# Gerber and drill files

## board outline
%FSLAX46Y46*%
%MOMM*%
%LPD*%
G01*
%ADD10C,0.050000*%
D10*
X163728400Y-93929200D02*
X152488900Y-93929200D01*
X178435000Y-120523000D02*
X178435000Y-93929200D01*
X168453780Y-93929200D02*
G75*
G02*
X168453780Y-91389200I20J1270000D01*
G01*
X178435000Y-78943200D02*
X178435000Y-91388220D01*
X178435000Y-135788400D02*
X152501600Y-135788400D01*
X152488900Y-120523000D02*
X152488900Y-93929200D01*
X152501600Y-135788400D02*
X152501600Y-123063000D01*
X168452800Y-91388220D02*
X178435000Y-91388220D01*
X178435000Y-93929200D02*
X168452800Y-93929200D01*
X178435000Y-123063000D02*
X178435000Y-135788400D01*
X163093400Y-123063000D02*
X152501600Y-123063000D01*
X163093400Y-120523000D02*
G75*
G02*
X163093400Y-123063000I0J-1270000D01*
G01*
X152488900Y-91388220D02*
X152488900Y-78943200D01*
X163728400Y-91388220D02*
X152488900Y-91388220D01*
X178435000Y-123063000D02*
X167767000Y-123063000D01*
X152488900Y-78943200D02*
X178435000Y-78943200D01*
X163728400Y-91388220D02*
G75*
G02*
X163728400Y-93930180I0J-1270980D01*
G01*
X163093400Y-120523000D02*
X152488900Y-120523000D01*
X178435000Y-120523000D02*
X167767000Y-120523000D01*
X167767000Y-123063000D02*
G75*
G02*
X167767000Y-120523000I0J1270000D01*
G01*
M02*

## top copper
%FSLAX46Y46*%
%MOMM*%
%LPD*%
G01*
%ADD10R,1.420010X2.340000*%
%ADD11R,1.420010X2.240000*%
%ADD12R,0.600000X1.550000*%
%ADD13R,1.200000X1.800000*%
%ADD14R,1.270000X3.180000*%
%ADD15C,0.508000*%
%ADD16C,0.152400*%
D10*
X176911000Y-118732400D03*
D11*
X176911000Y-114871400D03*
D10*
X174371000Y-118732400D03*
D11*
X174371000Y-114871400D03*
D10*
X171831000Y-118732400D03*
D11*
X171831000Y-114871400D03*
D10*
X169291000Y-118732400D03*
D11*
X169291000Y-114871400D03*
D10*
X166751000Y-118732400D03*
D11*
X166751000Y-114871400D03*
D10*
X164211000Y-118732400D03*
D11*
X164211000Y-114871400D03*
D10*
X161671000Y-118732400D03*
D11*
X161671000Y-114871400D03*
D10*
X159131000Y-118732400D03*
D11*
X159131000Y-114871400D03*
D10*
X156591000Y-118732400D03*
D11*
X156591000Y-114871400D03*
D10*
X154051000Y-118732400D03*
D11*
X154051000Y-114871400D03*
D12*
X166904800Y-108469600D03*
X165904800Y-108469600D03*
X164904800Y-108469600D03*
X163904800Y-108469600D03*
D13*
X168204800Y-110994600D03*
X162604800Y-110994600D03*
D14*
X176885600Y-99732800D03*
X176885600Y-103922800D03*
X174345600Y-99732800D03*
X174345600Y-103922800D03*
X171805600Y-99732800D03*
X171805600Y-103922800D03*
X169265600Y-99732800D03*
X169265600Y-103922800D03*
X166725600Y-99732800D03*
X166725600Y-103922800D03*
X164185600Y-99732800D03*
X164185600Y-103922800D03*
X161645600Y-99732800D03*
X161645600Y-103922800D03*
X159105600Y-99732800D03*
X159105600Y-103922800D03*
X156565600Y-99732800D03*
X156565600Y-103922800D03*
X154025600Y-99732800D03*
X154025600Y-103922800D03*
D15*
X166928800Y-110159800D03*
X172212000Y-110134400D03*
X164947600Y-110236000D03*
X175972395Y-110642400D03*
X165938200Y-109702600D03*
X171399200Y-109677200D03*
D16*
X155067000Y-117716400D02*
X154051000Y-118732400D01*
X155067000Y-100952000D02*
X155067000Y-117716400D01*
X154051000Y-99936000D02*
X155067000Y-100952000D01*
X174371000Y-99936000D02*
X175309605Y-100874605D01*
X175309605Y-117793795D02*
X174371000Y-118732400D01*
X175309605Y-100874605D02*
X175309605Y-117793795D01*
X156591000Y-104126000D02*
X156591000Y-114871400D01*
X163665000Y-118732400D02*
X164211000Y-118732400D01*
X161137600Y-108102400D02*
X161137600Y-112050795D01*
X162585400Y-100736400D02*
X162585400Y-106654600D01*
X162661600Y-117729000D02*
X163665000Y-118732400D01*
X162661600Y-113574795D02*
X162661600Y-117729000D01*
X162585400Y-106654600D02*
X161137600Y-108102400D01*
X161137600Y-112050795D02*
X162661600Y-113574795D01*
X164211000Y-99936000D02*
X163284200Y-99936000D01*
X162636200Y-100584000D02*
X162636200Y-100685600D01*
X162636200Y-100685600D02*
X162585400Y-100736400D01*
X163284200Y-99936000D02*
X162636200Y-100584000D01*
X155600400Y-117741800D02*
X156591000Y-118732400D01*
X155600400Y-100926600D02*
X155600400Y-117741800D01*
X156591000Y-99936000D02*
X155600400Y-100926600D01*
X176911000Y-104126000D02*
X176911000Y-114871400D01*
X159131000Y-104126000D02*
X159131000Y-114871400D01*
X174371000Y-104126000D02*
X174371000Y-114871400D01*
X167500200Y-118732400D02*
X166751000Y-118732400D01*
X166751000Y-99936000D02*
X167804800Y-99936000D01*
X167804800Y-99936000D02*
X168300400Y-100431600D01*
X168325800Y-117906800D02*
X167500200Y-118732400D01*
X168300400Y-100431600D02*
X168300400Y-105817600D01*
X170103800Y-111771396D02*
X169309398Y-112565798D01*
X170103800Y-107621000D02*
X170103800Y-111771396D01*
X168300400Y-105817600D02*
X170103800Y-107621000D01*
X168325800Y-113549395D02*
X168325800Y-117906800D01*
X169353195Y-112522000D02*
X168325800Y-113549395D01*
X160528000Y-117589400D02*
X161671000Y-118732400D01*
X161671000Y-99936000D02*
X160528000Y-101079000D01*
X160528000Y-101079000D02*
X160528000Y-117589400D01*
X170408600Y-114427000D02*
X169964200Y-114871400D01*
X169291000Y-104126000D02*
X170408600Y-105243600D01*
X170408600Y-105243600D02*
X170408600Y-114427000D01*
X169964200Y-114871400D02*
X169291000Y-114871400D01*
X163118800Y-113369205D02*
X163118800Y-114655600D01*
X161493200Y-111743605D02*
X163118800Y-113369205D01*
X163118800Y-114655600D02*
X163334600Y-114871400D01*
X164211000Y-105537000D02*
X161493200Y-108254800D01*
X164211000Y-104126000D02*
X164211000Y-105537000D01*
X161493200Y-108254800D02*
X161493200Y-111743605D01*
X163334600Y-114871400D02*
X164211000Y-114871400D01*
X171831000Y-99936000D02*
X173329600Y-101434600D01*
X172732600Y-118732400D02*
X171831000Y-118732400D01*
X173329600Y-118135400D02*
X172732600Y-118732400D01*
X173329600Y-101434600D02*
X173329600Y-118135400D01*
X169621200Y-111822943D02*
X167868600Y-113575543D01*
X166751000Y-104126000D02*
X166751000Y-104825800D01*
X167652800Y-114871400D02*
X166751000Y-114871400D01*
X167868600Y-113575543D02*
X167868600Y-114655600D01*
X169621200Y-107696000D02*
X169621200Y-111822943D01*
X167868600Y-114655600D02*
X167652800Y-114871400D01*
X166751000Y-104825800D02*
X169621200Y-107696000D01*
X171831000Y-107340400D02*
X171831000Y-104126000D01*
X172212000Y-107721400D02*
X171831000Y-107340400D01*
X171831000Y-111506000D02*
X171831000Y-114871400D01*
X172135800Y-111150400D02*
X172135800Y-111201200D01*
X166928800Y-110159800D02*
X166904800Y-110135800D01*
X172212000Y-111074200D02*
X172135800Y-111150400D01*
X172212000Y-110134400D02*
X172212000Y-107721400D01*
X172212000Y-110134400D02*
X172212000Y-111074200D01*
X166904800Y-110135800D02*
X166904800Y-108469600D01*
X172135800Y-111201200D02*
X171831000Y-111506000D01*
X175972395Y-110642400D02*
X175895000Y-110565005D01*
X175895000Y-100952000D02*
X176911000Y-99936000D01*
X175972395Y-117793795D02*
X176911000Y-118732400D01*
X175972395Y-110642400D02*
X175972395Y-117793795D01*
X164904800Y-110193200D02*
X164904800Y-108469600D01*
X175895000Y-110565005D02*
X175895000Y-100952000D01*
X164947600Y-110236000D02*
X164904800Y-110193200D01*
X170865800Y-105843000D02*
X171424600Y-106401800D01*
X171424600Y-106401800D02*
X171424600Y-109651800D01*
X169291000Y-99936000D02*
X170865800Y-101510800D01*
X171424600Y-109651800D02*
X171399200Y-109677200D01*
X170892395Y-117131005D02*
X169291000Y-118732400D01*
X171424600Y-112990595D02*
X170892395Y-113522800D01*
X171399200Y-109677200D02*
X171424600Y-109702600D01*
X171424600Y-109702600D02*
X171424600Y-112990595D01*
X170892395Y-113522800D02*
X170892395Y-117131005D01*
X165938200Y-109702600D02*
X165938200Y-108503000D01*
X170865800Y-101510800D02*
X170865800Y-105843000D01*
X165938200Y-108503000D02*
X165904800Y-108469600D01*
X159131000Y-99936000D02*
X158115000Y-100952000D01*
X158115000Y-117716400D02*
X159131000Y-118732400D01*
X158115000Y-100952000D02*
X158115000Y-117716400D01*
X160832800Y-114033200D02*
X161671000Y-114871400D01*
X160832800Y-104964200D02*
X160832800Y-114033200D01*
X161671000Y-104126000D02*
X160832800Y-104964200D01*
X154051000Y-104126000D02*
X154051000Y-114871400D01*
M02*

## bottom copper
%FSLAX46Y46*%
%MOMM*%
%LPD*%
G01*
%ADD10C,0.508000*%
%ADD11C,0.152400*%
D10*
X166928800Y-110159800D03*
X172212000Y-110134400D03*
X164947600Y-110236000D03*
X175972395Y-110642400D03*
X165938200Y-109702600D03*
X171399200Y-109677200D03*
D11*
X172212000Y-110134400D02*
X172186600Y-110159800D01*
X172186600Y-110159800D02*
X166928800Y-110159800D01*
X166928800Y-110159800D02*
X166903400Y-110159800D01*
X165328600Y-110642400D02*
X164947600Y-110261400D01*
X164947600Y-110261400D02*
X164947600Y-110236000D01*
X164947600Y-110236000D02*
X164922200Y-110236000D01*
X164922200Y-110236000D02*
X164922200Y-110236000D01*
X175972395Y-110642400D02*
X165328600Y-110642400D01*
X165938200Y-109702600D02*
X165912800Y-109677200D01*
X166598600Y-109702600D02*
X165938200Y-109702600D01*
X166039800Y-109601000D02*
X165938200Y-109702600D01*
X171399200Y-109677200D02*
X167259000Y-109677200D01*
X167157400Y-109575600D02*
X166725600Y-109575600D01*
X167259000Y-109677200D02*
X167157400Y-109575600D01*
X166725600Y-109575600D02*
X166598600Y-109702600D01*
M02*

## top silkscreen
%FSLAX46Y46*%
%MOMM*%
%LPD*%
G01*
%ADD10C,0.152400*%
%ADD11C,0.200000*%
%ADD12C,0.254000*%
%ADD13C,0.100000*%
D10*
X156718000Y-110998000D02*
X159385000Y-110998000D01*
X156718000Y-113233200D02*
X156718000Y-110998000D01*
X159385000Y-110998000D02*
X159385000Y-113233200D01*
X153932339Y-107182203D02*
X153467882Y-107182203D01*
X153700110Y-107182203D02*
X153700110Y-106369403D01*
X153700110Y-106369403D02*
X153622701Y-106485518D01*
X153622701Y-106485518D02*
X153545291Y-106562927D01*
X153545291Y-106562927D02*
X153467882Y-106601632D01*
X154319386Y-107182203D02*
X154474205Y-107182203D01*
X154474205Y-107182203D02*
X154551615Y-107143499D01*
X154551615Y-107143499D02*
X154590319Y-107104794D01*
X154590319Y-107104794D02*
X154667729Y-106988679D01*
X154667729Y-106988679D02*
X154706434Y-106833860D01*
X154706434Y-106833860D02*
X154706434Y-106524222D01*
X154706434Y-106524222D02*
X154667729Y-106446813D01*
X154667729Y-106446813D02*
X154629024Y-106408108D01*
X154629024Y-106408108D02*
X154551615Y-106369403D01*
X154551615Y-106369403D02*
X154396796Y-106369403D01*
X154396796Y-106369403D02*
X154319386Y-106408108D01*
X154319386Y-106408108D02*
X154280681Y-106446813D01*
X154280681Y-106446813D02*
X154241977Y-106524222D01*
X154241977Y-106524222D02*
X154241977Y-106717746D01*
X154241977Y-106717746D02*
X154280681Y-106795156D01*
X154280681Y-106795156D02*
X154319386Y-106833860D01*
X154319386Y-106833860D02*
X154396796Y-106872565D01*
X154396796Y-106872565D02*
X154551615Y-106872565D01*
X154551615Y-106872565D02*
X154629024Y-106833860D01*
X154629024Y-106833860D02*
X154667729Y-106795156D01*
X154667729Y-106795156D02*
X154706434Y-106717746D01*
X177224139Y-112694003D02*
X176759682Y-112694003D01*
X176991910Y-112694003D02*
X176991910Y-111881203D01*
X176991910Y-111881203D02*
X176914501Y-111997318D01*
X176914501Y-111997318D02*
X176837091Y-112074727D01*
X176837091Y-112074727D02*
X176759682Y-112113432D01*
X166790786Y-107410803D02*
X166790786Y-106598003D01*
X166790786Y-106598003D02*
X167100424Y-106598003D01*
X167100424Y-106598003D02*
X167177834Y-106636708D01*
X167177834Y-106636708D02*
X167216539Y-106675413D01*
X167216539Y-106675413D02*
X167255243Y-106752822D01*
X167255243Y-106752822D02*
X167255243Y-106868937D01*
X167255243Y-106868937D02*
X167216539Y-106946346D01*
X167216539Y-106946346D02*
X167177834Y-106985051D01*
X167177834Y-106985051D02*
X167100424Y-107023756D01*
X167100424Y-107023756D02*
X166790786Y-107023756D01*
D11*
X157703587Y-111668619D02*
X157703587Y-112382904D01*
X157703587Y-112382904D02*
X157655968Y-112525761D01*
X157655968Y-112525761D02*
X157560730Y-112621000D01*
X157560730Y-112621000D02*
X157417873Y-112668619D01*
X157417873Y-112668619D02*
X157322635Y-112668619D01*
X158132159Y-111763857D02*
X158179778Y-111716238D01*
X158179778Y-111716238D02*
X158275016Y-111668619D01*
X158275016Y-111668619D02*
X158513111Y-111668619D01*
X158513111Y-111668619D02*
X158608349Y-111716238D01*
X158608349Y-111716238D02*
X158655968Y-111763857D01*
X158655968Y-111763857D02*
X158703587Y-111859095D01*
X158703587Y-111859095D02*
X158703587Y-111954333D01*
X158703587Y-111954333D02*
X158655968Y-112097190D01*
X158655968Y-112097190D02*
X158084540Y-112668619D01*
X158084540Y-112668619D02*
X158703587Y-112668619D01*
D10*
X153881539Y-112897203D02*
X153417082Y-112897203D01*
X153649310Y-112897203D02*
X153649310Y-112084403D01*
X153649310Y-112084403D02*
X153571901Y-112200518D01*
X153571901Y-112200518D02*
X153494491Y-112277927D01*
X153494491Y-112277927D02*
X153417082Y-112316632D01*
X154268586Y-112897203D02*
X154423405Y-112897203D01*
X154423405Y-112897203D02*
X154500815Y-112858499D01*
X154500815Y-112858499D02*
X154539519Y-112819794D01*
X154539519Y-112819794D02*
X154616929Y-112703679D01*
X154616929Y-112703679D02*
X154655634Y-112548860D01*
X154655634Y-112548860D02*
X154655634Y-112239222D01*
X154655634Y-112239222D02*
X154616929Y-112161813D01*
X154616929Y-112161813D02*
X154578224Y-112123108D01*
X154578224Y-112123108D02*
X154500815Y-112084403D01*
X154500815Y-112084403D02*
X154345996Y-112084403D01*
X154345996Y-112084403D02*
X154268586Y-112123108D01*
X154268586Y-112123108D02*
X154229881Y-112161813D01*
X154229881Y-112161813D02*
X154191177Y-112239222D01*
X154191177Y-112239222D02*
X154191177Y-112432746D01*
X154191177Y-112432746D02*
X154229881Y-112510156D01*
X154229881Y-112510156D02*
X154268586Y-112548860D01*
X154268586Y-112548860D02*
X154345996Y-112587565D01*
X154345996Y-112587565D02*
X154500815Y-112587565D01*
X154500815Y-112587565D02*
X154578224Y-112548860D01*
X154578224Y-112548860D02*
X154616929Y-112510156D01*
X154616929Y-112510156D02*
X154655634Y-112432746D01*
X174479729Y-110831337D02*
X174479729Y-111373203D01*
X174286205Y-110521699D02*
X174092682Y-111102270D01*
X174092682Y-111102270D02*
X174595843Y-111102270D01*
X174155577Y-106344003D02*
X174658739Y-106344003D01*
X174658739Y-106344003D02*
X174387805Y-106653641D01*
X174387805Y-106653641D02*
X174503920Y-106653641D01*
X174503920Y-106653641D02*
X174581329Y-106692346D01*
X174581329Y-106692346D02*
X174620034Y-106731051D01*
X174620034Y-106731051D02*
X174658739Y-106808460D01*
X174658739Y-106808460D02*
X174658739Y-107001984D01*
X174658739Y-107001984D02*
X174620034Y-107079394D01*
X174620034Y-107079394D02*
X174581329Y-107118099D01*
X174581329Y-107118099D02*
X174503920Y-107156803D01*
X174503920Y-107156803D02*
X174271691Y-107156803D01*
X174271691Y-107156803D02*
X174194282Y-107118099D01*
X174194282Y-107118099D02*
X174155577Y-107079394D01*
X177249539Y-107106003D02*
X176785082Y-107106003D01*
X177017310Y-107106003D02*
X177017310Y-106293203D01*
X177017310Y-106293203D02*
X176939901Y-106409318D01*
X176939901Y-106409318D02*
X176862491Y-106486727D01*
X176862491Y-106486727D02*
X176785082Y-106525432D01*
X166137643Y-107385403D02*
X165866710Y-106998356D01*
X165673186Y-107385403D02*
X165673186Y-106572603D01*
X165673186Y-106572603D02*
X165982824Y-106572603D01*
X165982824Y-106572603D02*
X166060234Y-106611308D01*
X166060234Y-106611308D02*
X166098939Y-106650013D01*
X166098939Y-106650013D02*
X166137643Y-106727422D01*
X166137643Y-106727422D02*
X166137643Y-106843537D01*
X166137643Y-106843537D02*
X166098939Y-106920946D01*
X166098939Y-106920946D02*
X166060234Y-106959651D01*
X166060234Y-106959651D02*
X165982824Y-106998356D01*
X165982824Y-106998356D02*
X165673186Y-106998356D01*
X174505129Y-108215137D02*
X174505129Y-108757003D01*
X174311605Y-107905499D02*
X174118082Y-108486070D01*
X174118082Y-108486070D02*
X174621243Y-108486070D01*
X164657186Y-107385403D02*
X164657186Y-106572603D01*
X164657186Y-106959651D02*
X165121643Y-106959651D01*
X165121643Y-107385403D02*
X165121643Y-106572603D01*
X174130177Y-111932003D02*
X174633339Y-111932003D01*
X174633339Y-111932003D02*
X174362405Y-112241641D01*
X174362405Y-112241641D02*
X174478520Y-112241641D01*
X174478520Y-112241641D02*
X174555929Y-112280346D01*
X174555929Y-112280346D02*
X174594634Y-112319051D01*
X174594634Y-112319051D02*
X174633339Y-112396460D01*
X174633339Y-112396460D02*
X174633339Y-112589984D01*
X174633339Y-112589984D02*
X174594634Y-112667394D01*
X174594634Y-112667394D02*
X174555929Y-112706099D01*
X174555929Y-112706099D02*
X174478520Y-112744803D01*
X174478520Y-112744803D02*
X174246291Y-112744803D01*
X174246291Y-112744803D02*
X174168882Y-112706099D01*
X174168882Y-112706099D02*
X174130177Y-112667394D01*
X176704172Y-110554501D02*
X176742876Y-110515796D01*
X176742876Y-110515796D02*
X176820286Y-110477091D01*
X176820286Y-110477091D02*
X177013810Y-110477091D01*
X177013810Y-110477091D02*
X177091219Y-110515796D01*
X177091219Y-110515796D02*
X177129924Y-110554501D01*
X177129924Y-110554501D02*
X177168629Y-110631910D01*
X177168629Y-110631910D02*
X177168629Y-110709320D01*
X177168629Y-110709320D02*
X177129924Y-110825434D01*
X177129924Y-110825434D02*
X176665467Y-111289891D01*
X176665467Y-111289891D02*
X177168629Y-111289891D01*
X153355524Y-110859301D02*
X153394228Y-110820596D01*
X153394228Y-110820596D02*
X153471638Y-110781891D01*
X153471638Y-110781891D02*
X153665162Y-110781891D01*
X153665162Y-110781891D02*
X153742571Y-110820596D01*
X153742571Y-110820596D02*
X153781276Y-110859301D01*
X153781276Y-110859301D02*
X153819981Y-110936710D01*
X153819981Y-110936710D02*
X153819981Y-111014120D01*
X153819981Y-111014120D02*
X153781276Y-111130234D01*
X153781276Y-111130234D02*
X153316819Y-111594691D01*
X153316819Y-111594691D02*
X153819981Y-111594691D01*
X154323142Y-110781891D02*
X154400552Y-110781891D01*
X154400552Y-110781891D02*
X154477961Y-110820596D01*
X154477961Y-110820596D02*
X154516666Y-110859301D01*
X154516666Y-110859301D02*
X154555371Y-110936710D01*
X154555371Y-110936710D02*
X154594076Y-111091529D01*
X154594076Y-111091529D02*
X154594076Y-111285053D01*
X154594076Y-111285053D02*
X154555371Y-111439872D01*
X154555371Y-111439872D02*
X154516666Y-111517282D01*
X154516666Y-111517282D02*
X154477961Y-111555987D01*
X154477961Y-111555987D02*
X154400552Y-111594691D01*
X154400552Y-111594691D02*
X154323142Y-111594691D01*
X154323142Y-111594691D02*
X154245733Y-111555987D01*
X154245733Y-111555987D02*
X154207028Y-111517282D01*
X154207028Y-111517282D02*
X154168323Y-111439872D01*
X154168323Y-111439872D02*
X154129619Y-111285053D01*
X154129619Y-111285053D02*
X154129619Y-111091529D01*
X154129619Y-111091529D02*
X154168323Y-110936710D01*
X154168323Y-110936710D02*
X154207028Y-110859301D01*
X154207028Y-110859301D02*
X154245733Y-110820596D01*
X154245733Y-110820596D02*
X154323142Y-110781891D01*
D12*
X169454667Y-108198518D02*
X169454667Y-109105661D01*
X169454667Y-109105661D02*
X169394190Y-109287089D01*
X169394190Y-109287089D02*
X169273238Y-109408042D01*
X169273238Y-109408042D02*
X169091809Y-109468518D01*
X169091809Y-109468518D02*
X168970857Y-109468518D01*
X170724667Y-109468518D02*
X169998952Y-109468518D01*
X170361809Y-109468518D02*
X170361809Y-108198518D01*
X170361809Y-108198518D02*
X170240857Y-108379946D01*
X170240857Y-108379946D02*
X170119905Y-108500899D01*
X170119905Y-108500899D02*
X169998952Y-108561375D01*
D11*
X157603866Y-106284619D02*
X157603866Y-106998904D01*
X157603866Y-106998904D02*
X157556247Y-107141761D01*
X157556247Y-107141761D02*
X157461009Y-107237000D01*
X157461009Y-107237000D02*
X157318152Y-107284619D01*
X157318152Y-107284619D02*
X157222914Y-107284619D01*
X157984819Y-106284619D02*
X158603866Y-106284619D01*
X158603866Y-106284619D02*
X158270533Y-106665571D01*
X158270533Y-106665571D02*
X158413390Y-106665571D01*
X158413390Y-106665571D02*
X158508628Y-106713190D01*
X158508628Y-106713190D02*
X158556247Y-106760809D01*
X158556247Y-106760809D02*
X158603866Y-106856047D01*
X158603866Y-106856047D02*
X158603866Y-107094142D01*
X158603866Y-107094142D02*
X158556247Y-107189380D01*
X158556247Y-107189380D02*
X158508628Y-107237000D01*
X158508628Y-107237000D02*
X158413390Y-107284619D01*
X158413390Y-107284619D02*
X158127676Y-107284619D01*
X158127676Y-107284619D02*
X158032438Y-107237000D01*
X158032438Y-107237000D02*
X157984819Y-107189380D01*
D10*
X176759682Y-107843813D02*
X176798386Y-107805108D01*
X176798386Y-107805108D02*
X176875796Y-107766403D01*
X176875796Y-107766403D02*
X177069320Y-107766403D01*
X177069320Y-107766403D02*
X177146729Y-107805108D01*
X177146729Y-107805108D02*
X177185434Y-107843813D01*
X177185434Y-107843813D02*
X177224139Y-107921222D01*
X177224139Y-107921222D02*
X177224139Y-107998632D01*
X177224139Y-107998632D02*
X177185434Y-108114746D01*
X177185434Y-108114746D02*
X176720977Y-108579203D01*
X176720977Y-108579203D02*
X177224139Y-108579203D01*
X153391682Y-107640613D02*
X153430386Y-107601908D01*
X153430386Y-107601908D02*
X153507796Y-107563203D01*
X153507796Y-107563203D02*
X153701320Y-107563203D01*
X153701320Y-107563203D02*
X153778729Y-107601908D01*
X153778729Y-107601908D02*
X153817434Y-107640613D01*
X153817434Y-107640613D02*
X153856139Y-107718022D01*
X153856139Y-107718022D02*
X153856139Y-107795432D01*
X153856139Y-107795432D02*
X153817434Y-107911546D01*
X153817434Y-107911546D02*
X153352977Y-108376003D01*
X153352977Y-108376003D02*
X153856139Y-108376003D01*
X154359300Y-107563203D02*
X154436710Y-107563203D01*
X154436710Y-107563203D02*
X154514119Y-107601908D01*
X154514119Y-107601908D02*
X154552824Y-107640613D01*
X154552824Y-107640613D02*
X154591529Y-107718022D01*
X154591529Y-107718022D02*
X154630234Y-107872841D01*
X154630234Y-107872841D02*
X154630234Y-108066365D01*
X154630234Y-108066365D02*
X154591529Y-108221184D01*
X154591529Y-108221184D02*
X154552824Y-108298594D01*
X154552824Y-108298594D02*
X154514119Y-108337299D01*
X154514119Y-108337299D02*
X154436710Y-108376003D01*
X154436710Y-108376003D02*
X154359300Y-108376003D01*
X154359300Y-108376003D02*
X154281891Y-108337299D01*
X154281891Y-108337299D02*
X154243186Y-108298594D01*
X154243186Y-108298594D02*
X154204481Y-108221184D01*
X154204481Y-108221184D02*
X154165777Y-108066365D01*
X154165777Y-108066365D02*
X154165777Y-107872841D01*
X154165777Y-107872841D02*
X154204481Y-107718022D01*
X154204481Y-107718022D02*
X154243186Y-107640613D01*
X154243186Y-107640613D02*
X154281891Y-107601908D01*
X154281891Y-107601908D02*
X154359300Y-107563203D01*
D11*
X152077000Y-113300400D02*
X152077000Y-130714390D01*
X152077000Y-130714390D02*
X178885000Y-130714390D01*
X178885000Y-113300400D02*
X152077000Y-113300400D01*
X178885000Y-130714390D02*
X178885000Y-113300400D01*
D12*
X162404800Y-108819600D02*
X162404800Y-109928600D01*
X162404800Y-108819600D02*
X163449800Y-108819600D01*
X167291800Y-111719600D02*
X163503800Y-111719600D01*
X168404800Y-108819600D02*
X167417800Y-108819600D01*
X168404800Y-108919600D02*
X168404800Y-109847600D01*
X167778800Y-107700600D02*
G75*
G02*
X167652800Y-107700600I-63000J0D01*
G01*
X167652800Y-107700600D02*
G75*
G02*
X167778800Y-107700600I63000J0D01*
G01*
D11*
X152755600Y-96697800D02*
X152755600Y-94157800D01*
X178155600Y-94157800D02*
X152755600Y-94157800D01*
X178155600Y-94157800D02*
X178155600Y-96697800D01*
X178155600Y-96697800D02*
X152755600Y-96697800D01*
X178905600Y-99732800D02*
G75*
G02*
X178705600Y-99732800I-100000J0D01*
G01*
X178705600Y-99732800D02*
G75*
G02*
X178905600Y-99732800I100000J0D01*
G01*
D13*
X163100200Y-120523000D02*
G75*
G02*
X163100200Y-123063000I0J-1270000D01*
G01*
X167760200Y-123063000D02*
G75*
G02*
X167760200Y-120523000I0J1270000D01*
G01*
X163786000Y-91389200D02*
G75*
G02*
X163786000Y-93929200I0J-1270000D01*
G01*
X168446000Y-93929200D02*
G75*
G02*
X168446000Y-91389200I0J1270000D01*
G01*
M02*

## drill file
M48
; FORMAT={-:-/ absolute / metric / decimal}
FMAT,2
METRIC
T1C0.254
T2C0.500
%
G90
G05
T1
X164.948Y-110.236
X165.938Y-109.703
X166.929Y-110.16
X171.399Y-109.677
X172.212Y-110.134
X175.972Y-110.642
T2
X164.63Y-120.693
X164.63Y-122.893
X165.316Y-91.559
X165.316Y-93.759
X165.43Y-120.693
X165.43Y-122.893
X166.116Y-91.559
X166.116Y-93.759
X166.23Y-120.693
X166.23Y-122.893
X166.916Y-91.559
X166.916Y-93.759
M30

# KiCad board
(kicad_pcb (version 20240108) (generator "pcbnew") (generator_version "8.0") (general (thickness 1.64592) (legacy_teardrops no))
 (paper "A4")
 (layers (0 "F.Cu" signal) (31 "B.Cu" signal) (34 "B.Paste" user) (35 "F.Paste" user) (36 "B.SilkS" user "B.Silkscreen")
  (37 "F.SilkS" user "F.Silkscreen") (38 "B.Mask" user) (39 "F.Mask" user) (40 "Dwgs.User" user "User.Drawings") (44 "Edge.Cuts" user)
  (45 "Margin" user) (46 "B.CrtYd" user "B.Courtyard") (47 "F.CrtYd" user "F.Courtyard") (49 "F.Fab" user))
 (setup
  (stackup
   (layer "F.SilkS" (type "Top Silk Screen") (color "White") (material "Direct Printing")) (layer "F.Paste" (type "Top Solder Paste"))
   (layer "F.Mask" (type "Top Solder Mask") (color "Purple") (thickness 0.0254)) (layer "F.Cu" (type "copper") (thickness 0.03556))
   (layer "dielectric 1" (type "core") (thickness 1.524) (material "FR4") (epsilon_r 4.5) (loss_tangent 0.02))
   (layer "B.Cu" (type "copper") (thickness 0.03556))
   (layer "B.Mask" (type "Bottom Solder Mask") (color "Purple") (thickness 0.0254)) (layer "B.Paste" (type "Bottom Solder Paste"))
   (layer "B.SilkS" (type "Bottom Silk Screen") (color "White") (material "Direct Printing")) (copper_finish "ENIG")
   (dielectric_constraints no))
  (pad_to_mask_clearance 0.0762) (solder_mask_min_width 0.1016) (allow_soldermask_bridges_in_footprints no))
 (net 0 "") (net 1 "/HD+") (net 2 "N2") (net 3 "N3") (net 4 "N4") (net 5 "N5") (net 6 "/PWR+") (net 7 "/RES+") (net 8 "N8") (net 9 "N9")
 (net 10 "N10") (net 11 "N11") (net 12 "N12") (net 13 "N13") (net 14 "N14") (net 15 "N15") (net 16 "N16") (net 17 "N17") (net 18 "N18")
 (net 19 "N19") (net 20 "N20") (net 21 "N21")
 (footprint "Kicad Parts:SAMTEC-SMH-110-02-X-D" (layer "F.Cu") (at 165.481 126.0094 180)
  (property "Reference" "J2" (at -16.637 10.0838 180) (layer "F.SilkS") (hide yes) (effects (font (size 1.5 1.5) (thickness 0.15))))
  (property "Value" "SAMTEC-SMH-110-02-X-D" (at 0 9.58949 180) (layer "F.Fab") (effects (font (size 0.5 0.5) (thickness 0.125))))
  (fp_line (start 13.404 12.709) (end 13.404 -4.70499) (stroke (width 0.2) (type solid)) (layer "F.SilkS"))
  (fp_line (start 13.404 -4.70499) (end -13.404 -4.70499) (stroke (width 0.2) (type solid)) (layer "F.SilkS"))
  (fp_line (start -13.404 12.709) (end 13.404 12.709) (stroke (width 0.2) (type solid)) (layer "F.SilkS"))
  (fp_line (start -13.404 -4.70499) (end -13.404 12.709) (stroke (width 0.2) (type solid)) (layer "F.SilkS"))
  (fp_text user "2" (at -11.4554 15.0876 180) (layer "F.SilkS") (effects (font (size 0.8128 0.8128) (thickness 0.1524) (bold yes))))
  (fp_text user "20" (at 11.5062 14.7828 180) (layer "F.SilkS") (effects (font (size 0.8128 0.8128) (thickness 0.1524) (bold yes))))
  (pad "1" smd rect (at -11.43 7.277 180) (size 1.42001 2.34) (layers "F.Cu" "F.Paste") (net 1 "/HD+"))
  (pad "2" smd rect (at -11.43 11.138 180) (size 1.42001 2.24) (layers "F.Cu" "F.Paste") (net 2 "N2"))
  (pad "3" smd rect (at -8.89 7.277 180) (size 1.42001 2.34) (layers "F.Cu" "F.Paste") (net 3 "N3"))
  (pad "4" smd rect (at -8.89 11.138 180) (size 1.42001 2.24) (layers "F.Cu" "F.Paste") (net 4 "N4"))
  (pad "5" smd rect (at -6.35 7.277 180) (size 1.42001 2.34) (layers "F.Cu" "F.Paste") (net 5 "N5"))
  (pad "6" smd rect (at -6.35 11.138 180) (size 1.42001 2.24) (layers "F.Cu" "F.Paste") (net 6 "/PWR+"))
  (pad "7" smd rect (at -3.81 7.277 180) (size 1.42001 2.34) (layers "F.Cu" "F.Paste") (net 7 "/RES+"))
  (pad "8" smd rect (at -3.81 11.138 180) (size 1.42001 2.24) (layers "F.Cu" "F.Paste") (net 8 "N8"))
  (pad "9" smd rect (at -1.27 7.277 180) (size 1.42001 2.34) (layers "F.Cu" "F.Paste") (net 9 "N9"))
  (pad "10" smd rect (at -1.27 11.138 180) (size 1.42001 2.24) (layers "F.Cu" "F.Paste") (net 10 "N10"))
  (pad "11" smd rect (at 1.27 7.277 180) (size 1.42001 2.34) (layers "F.Cu" "F.Paste") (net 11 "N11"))
  (pad "12" smd rect (at 1.27 11.138 180) (size 1.42001 2.24) (layers "F.Cu" "F.Paste") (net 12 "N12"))
  (pad "13" smd rect (at 3.81 7.277 180) (size 1.42001 2.34) (layers "F.Cu" "F.Paste") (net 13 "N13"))
  (pad "14" smd rect (at 3.81 11.138 180) (size 1.42001 2.24) (layers "F.Cu" "F.Paste") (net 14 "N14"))
  (pad "15" smd rect (at 6.35 7.277 180) (size 1.42001 2.34) (layers "F.Cu" "F.Paste") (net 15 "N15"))
  (pad "16" smd rect (at 6.35 11.138 180) (size 1.42001 2.24) (layers "F.Cu" "F.Paste") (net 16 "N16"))
  (pad "17" smd rect (at 8.89 7.277 180) (size 1.42001 2.34) (layers "F.Cu" "F.Paste") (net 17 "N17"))
  (pad "18" smd rect (at 8.89 11.138 180) (size 1.42001 2.24) (layers "F.Cu" "F.Paste") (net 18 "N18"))
  (pad "19" smd rect (at 11.43 7.277 180) (size 1.42001 2.34) (layers "F.Cu" "F.Paste") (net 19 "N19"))
  (pad "20" smd rect (at 11.43 11.138 180) (size 1.42001 2.24) (layers "F.Cu" "F.Paste") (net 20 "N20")))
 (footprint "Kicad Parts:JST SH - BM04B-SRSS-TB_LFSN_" (layer "F.Cu") (at 168.4048 108.9196 180)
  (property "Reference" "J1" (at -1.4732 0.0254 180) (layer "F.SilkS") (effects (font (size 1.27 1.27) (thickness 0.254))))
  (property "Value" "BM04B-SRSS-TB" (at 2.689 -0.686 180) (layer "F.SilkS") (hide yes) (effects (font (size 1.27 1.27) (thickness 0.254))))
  (fp_line (start 6 0.1) (end 6 -1.009) (stroke (width 0.254) (type solid)) (layer "F.SilkS"))
  (fp_line (start 6 0.1) (end 4.955 0.1) (stroke (width 0.254) (type solid)) (layer "F.SilkS"))
  (fp_line (start 1.113 -2.8) (end 4.901 -2.8) (stroke (width 0.254) (type solid)) (layer "F.SilkS"))
  (fp_line (start 0 0.1) (end 0.987 0.1) (stroke (width 0.254) (type solid)) (layer "F.SilkS"))
  (fp_line (start 0 0) (end 0 -0.928) (stroke (width 0.254) (type solid)) (layer "F.SilkS"))
  (fp_circle (center 0.689 1.219) (end 0.689 1.282) (stroke (width 0.254) (type solid)) (fill none) (layer "F.SilkS"))
  (pad "1" smd rect (at 1.5 0.45 180) (size 0.6 1.55) (layers "F.Cu" "F.Paste" "F.Mask") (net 6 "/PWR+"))
  (pad "2" smd rect (at 2.5 0.45 180) (size 0.6 1.55) (layers "F.Cu" "F.Paste" "F.Mask") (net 7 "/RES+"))
  (pad "3" smd rect (at 3.5 0.45 180) (size 0.6 1.55) (layers "F.Cu" "F.Paste" "F.Mask") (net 1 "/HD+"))
  (pad "4" smd rect (at 4.5 0.45 180) (size 0.6 1.55) (layers "F.Cu" "F.Paste" "F.Mask") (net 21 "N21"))
  (pad "5" smd rect (at 0.2 -2.075 180) (size 1.2 1.8) (layers "F.Cu" "F.Paste" "F.Mask"))
  (pad "6" smd rect (at 5.8 -2.075 180) (size 1.2 1.8) (layers "F.Cu" "F.Paste" "F.Mask")))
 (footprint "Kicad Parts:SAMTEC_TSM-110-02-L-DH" (layer "F.Cu") (at 165.4556 95.4278)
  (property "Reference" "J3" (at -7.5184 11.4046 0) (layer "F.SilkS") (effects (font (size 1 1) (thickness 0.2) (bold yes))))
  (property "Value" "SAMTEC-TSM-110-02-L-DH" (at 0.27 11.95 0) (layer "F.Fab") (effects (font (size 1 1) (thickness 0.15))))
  (fp_line (start -12.7 1.27) (end -12.7 -1.27) (stroke (width 0.2) (type solid)) (layer "F.SilkS"))
  (fp_line (start 12.7 -1.27) (end -12.7 -1.27) (stroke (width 0.2) (type solid)) (layer "F.SilkS"))
  (fp_line (start 12.7 -1.27) (end 12.7 1.27) (stroke (width 0.2) (type solid)) (layer "F.SilkS"))
  (fp_line (start 12.7 1.27) (end -12.7 1.27) (stroke (width 0.2) (type solid)) (layer "F.SilkS"))
  (fp_circle (center 13.35 4.305) (end 13.45 4.305) (stroke (width 0.2) (type solid)) (fill none) (layer "F.SilkS"))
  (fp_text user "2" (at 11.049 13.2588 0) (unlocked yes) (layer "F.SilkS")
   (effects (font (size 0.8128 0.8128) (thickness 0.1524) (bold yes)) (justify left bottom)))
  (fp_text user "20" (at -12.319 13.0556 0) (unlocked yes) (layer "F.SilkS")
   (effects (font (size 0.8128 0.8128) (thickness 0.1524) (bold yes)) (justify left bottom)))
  (pad "01" smd rect (at 11.43 4.305) (size 1.27 3.18) (layers "F.Cu" "F.Paste" "F.Mask") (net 1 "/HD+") (solder_mask_margin 0.102))
  (pad "02" smd rect (at 11.43 8.495) (size 1.27 3.18) (layers "F.Cu" "F.Paste" "F.Mask") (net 2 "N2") (solder_mask_margin 0.102))
  (pad "03" smd rect (at 8.89 4.305) (size 1.27 3.18) (layers "F.Cu" "F.Paste" "F.Mask") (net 3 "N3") (solder_mask_margin 0.102))
  (pad "04" smd rect (at 8.89 8.495) (size 1.27 3.18) (layers "F.Cu" "F.Paste" "F.Mask") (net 4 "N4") (solder_mask_margin 0.102))
  (pad "05" smd rect (at 6.35 4.305) (size 1.27 3.18) (layers "F.Cu" "F.Paste" "F.Mask") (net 5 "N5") (solder_mask_margin 0.102))
  (pad "06" smd rect (at 6.35 8.495) (size 1.27 3.18) (layers "F.Cu" "F.Paste" "F.Mask") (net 6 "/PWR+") (solder_mask_margin 0.102))
  (pad "07" smd rect (at 3.81 4.305) (size 1.27 3.18) (layers "F.Cu" "F.Paste" "F.Mask") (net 7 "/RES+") (solder_mask_margin 0.102))
  (pad "08" smd rect (at 3.81 8.495) (size 1.27 3.18) (layers "F.Cu" "F.Paste" "F.Mask") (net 8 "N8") (solder_mask_margin 0.102))
  (pad "09" smd rect (at 1.27 4.305) (size 1.27 3.18) (layers "F.Cu" "F.Paste" "F.Mask") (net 9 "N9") (solder_mask_margin 0.102))
  (pad "10" smd rect (at 1.27 8.495) (size 1.27 3.18) (layers "F.Cu" "F.Paste" "F.Mask") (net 10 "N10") (solder_mask_margin 0.102))
  (pad "11" smd rect (at -1.27 4.305) (size 1.27 3.18) (layers "F.Cu" "F.Paste" "F.Mask") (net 11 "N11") (solder_mask_margin 0.102))
  (pad "12" smd rect (at -1.27 8.495) (size 1.27 3.18) (layers "F.Cu" "F.Paste" "F.Mask") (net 12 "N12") (solder_mask_margin 0.102))
  (pad "13" smd rect (at -3.81 4.305) (size 1.27 3.18) (layers "F.Cu" "F.Paste" "F.Mask") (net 13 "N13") (solder_mask_margin 0.102))
  (pad "14" smd rect (at -3.81 8.495) (size 1.27 3.18) (layers "F.Cu" "F.Paste" "F.Mask") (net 14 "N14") (solder_mask_margin 0.102))
  (pad "15" smd rect (at -6.35 4.305) (size 1.27 3.18) (layers "F.Cu" "F.Paste" "F.Mask") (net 15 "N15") (solder_mask_margin 0.102))
  (pad "16" smd rect (at -6.35 8.495) (size 1.27 3.18) (layers "F.Cu" "F.Paste" "F.Mask") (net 16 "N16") (solder_mask_margin 0.102))
  (pad "17" smd rect (at -8.89 4.305) (size 1.27 3.18) (layers "F.Cu" "F.Paste" "F.Mask") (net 17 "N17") (solder_mask_margin 0.102))
  (pad "18" smd rect (at -8.89 8.495) (size 1.27 3.18) (layers "F.Cu" "F.Paste" "F.Mask") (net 18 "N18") (solder_mask_margin 0.102))
  (pad "19" smd rect (at -11.43 4.305) (size 1.27 3.18) (layers "F.Cu" "F.Paste" "F.Mask") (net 19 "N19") (solder_mask_margin 0.102))
  (pad "20" smd rect (at -11.43 8.495) (size 1.27 3.18) (layers "F.Cu" "F.Paste" "F.Mask") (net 20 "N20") (solder_mask_margin 0.102)))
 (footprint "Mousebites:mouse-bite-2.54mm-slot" (layer "F.Cu") (at 165.4302 121.793)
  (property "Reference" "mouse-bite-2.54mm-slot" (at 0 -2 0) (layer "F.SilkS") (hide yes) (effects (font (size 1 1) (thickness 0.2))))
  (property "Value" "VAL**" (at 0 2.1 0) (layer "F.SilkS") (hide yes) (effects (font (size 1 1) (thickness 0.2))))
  (fp_arc (start -2.33 -1.27) (mid -1.06 0) (end -2.33 1.27) (stroke (width 0.1) (type solid)) (layer "F.SilkS"))
  (fp_arc (start 2.33 1.27) (mid 1.06 0) (end 2.33 -1.27) (stroke (width 0.1) (type solid)) (layer "F.SilkS"))
  (pad "" np_thru_hole circle (at -0.8 -1.1) (size 0.5 0.5) (drill 0.5) (layers "*.Cu" "*.Mask"))
  (pad "" np_thru_hole circle (at -0.8 1.1) (size 0.5 0.5) (drill 0.5) (layers "*.Cu" "*.Mask"))
  (pad "" np_thru_hole circle (at 0 -1.1) (size 0.5 0.5) (drill 0.5) (layers "*.Cu" "*.Mask"))
  (pad "" np_thru_hole circle (at 0 1.1) (size 0.5 0.5) (drill 0.5) (layers "*.Cu" "*.Mask"))
  (pad "" np_thru_hole circle (at 0.8 -1.1) (size 0.5 0.5) (drill 0.5) (layers "*.Cu" "*.Mask"))
  (pad "" np_thru_hole circle (at 0.8 1.1) (size 0.5 0.5) (drill 0.5) (layers "*.Cu" "*.Mask")))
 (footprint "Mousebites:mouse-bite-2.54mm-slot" (layer "F.Cu") (at 166.116 92.6592)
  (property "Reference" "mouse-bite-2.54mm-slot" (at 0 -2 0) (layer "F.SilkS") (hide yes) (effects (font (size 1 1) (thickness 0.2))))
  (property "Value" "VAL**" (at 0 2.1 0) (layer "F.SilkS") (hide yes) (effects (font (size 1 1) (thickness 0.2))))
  (fp_arc (start -2.33 -1.27) (mid -1.06 0) (end -2.33 1.27) (stroke (width 0.1) (type solid)) (layer "F.SilkS"))
  (fp_arc (start 2.33 1.27) (mid 1.06 0) (end 2.33 -1.27) (stroke (width 0.1) (type solid)) (layer "F.SilkS"))
  (pad "" np_thru_hole circle (at -0.8 -1.1) (size 0.5 0.5) (drill 0.5) (layers "*.Cu" "*.Mask"))
  (pad "" np_thru_hole circle (at -0.8 1.1) (size 0.5 0.5) (drill 0.5) (layers "*.Cu" "*.Mask"))
  (pad "" np_thru_hole circle (at 0 -1.1) (size 0.5 0.5) (drill 0.5) (layers "*.Cu" "*.Mask"))
  (pad "" np_thru_hole circle (at 0 1.1) (size 0.5 0.5) (drill 0.5) (layers "*.Cu" "*.Mask"))
  (pad "" np_thru_hole circle (at 0.8 -1.1) (size 0.5 0.5) (drill 0.5) (layers "*.Cu" "*.Mask"))
  (pad "" np_thru_hole circle (at 0.8 1.1) (size 0.5 0.5) (drill 0.5) (layers "*.Cu" "*.Mask")))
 (gr_line (start 156.718 110.998) (end 159.385 110.998) (stroke (width 0.1524) (type default)) (layer "F.SilkS"))
 (gr_line (start 156.718 113.2332) (end 156.718 110.998) (stroke (width 0.1524) (type default)) (layer "F.SilkS"))
 (gr_line (start 159.385 110.998) (end 159.385 113.2332) (stroke (width 0.1524) (type default)) (layer "F.SilkS"))
 (gr_line (start 163.7284 93.9292) (end 152.4889 93.9292) (stroke (width 0.05) (type default)) (layer "Edge.Cuts"))
 (gr_line (start 178.435 120.523) (end 178.435 93.9292) (stroke (width 0.05) (type default)) (layer "Edge.Cuts"))
 (gr_arc (start 168.45378 93.9292) (mid 167.18378 92.6592) (end 168.45378 91.3892) (stroke (width 0.05) (type default)) (layer "Edge.Cuts"))
 (gr_line (start 178.435 78.9432) (end 178.435 91.38822) (stroke (width 0.05) (type default)) (layer "Edge.Cuts"))
 (gr_line (start 178.435 135.7884) (end 152.5016 135.7884) (stroke (width 0.05) (type default)) (layer "Edge.Cuts"))
 (gr_line (start 152.4889 120.523) (end 152.4889 93.9292) (stroke (width 0.05) (type default)) (layer "Edge.Cuts"))
 (gr_line (start 152.5016 135.7884) (end 152.5016 123.063) (stroke (width 0.05) (type default)) (layer "Edge.Cuts"))
 (gr_line (start 168.4528 91.38822) (end 178.435 91.38822) (stroke (width 0.05) (type default)) (layer "Edge.Cuts"))
 (gr_line (start 178.435 93.9292) (end 168.4528 93.9292) (stroke (width 0.05) (type default)) (layer "Edge.Cuts"))
 (gr_line (start 178.435 123.063) (end 178.435 135.7884) (stroke (width 0.05) (type default)) (layer "Edge.Cuts"))
 (gr_line (start 163.0934 123.063) (end 152.5016 123.063) (stroke (width 0.05) (type default)) (layer "Edge.Cuts"))
 (gr_arc (start 163.0934 120.523) (mid 164.3634 121.793) (end 163.0934 123.063) (stroke (width 0.05) (type default)) (layer "Edge.Cuts"))
 (gr_line (start 152.4889 91.38822) (end 152.4889 78.9432) (stroke (width 0.05) (type default)) (layer "Edge.Cuts"))
 (gr_line (start 163.7284 91.38822) (end 152.4889 91.38822) (stroke (width 0.05) (type default)) (layer "Edge.Cuts"))
 (gr_line (start 178.435 123.063) (end 167.767 123.063) (stroke (width 0.05) (type default)) (layer "Edge.Cuts"))
 (gr_line (start 152.4889 78.9432) (end 178.435 78.9432) (stroke (width 0.05) (type default)) (layer "Edge.Cuts"))
 (gr_arc (start 163.7284 91.38822) (mid 164.99938 92.6592) (end 163.7284 93.93018) (stroke (width 0.05) (type default)) (layer "Edge.Cuts"))
 (gr_line (start 163.0934 120.523) (end 152.4889 120.523) (stroke (width 0.05) (type default)) (layer "Edge.Cuts"))
 (gr_line (start 178.435 120.523) (end 167.767 120.523) (stroke (width 0.05) (type default)) (layer "Edge.Cuts"))
 (gr_arc (start 167.767 123.063) (mid 166.497 121.793) (end 167.767 120.523) (stroke (width 0.05) (type default)) (layer "Edge.Cuts"))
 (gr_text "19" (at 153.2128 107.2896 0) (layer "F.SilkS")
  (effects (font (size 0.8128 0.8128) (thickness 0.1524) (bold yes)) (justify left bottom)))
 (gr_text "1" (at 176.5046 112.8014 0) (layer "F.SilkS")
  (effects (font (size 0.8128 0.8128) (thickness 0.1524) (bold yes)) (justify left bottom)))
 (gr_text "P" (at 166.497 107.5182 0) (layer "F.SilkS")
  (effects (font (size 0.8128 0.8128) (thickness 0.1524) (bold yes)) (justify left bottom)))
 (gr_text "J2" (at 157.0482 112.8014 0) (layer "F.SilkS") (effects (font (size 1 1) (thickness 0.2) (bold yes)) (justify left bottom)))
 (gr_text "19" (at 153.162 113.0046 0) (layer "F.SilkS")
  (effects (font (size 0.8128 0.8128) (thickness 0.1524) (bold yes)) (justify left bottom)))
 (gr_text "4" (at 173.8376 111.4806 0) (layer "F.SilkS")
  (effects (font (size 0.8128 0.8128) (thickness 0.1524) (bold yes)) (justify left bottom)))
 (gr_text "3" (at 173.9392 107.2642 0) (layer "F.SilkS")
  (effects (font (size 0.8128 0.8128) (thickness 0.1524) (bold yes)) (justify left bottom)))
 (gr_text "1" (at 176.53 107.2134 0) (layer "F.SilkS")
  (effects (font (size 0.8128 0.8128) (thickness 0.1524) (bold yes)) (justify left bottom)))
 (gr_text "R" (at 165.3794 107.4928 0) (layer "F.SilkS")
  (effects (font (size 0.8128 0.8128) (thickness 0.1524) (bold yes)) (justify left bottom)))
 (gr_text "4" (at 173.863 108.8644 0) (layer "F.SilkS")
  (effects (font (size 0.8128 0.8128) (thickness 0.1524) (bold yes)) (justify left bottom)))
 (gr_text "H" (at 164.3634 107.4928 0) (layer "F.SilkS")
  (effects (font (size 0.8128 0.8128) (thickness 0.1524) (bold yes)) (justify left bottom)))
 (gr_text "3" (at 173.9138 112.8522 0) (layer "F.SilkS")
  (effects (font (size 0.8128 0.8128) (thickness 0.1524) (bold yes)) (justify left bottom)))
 (segment (start 155.067 117.7164) (end 154.051 118.7324) (width 0.1524) (layer "F.Cu") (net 19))
 (segment (start 155.067 100.952) (end 155.067 117.7164) (width 0.1524) (layer "F.Cu") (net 19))
 (segment (start 154.051 99.936) (end 155.067 100.952) (width 0.1524) (layer "F.Cu") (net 19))
 (segment (start 174.371 99.936) (end 175.309605 100.874605) (width 0.1524) (layer "F.Cu") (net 3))
 (segment (start 175.309605 117.793795) (end 174.371 118.7324) (width 0.1524) (layer "F.Cu") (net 3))
 (segment (start 175.309605 100.874605) (end 175.309605 117.793795) (width 0.1524) (layer "F.Cu") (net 3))
 (segment (start 156.591 104.126) (end 156.591 114.8714) (width 0.1524) (layer "F.Cu") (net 18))
 (segment (start 163.665 118.7324) (end 164.211 118.7324) (width 0.1524) (layer "F.Cu") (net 11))
 (segment (start 161.1376 108.1024) (end 161.1376 112.050795) (width 0.1524) (layer "F.Cu") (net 11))
 (segment (start 162.5854 100.7364) (end 162.5854 106.6546) (width 0.1524) (layer "F.Cu") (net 11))
 (segment (start 162.6616 117.729) (end 163.665 118.7324) (width 0.1524) (layer "F.Cu") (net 11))
 (segment (start 162.6616 113.574795) (end 162.6616 117.729) (width 0.1524) (layer "F.Cu") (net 11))
 (segment (start 162.5854 106.6546) (end 161.1376 108.1024) (width 0.1524) (layer "F.Cu") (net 11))
 (segment (start 161.1376 112.050795) (end 162.6616 113.574795) (width 0.1524) (layer "F.Cu") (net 11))
 (segment (start 164.211 99.936) (end 163.2842 99.936) (width 0.1524) (layer "F.Cu") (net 11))
 (segment (start 162.6362 100.584) (end 162.6362 100.6856) (width 0.1524) (layer "F.Cu") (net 11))
 (segment (start 162.6362 100.6856) (end 162.5854 100.7364) (width 0.1524) (layer "F.Cu") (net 11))
 (segment (start 163.2842 99.936) (end 162.6362 100.584) (width 0.1524) (layer "F.Cu") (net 11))
 (segment (start 155.6004 117.7418) (end 156.591 118.7324) (width 0.1524) (layer "F.Cu") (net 17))
 (segment (start 155.6004 100.9266) (end 155.6004 117.7418) (width 0.1524) (layer "F.Cu") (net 17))
 (segment (start 156.591 99.936) (end 155.6004 100.9266) (width 0.1524) (layer "F.Cu") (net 17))
 (segment (start 176.911 104.126) (end 176.911 114.8714) (width 0.1524) (layer "F.Cu") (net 2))
 (segment (start 159.131 104.126) (end 159.131 114.8714) (width 0.1524) (layer "F.Cu") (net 16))
 (segment (start 174.371 104.126) (end 174.371 114.8714) (width 0.1524) (layer "F.Cu") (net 4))
 (segment (start 167.5002 118.7324) (end 166.751 118.7324) (width 0.1524) (layer "F.Cu") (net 9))
 (segment (start 166.751 99.936) (end 167.8048 99.936) (width 0.1524) (layer "F.Cu") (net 9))
 (segment (start 167.8048 99.936) (end 168.3004 100.4316) (width 0.1524) (layer "F.Cu") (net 9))
 (segment (start 168.3258 117.9068) (end 167.5002 118.7324) (width 0.1524) (layer "F.Cu") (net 9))
 (segment (start 168.3004 100.4316) (end 168.3004 105.8176) (width 0.1524) (layer "F.Cu") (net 9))
 (segment (start 170.1038 111.771396) (end 169.309398 112.565798) (width 0.1524) (layer "F.Cu") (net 9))
 (segment (start 170.1038 107.621) (end 170.1038 111.771396) (width 0.1524) (layer "F.Cu") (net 9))
 (segment (start 168.3004 105.8176) (end 170.1038 107.621) (width 0.1524) (layer "F.Cu") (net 9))
 (segment (start 168.3258 113.549395) (end 168.3258 117.9068) (width 0.1524) (layer "F.Cu") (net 9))
 (segment (start 169.353195 112.522) (end 168.3258 113.549395) (width 0.1524) (layer "F.Cu") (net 9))
 (segment (start 160.528 117.5894) (end 161.671 118.7324) (width 0.1524) (layer "F.Cu") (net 13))
 (segment (start 161.671 99.936) (end 160.528 101.079) (width 0.1524) (layer "F.Cu") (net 13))
 (segment (start 160.528 101.079) (end 160.528 117.5894) (width 0.1524) (layer "F.Cu") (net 13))
 (segment (start 170.4086 114.427) (end 169.9642 114.8714) (width 0.1524) (layer "F.Cu") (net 8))
 (segment (start 169.291 104.126) (end 170.4086 105.2436) (width 0.1524) (layer "F.Cu") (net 8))
 (segment (start 170.4086 105.2436) (end 170.4086 114.427) (width 0.1524) (layer "F.Cu") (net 8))
 (segment (start 169.9642 114.8714) (end 169.291 114.8714) (width 0.1524) (layer "F.Cu") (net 8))
 (segment (start 163.1188 113.369205) (end 163.1188 114.6556) (width 0.1524) (layer "F.Cu") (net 12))
 (segment (start 161.4932 111.743605) (end 163.1188 113.369205) (width 0.1524) (layer "F.Cu") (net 12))
 (segment (start 163.1188 114.6556) (end 163.3346 114.8714) (width 0.1524) (layer "F.Cu") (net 12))
 (segment (start 164.211 105.537) (end 161.4932 108.2548) (width 0.1524) (layer "F.Cu") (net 12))
 (segment (start 164.211 104.126) (end 164.211 105.537) (width 0.1524) (layer "F.Cu") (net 12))
 (segment (start 161.4932 108.2548) (end 161.4932 111.743605) (width 0.1524) (layer "F.Cu") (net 12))
 (segment (start 163.3346 114.8714) (end 164.211 114.8714) (width 0.1524) (layer "F.Cu") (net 12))
 (segment (start 171.831 99.936) (end 173.3296 101.4346) (width 0.1524) (layer "F.Cu") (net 5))
 (segment (start 172.7326 118.7324) (end 171.831 118.7324) (width 0.1524) (layer "F.Cu") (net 5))
 (segment (start 173.3296 118.1354) (end 172.7326 118.7324) (width 0.1524) (layer "F.Cu") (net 5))
 (segment (start 173.3296 101.4346) (end 173.3296 118.1354) (width 0.1524) (layer "F.Cu") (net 5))
 (segment (start 169.6212 111.822943) (end 167.8686 113.575543) (width 0.1524) (layer "F.Cu") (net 10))
 (segment (start 166.751 104.126) (end 166.751 104.8258) (width 0.1524) (layer "F.Cu") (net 10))
 (segment (start 167.6528 114.8714) (end 166.751 114.8714) (width 0.1524) (layer "F.Cu") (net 10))
 (segment (start 167.8686 113.575543) (end 167.8686 114.6556) (width 0.1524) (layer "F.Cu") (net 10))
 (segment (start 169.6212 107.696) (end 169.6212 111.822943) (width 0.1524) (layer "F.Cu") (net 10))
 (segment (start 167.8686 114.6556) (end 167.6528 114.8714) (width 0.1524) (layer "F.Cu") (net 10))
 (segment (start 166.751 104.8258) (end 169.6212 107.696) (width 0.1524) (layer "F.Cu") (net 10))
 (segment (start 171.831 107.3404) (end 171.831 104.126) (width 0.1524) (layer "F.Cu") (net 6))
 (segment (start 172.212 107.7214) (end 171.831 107.3404) (width 0.1524) (layer "F.Cu") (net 6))
 (segment (start 171.831 111.506) (end 171.831 114.8714) (width 0.1524) (layer "F.Cu") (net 6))
 (segment (start 172.1358 111.1504) (end 172.1358 111.2012) (width 0.1524) (layer "F.Cu") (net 6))
 (segment (start 166.9288 110.1598) (end 166.9048 110.1358) (width 0.1524) (layer "F.Cu") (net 6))
 (segment (start 172.212 111.0742) (end 172.1358 111.1504) (width 0.1524) (layer "F.Cu") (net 6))
 (segment (start 172.212 110.1344) (end 172.212 107.7214) (width 0.1524) (layer "F.Cu") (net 6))
 (segment (start 172.212 110.1344) (end 172.212 111.0742) (width 0.1524) (layer "F.Cu") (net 6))
 (segment (start 166.9048 110.1358) (end 166.9048 108.4696) (width 0.1524) (layer "F.Cu") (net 6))
 (segment (start 172.1358 111.2012) (end 171.831 111.506) (width 0.1524) (layer "F.Cu") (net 6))
 (via (at 166.9288 110.1598) (size 0.508) (drill 0.254) (layers "F.Cu" "B.Cu") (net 6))
 (via (at 172.212 110.1344) (size 0.508) (drill 0.254) (layers "F.Cu" "B.Cu") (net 6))
 (segment (start 172.212 110.1344) (end 172.1866 110.1598) (width 0.1524) (layer "B.Cu") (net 6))
 (segment (start 172.1866 110.1598) (end 166.9288 110.1598) (width 0.1524) (layer "B.Cu") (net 6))
 (segment (start 166.9288 110.1598) (end 166.9034 110.1598) (width 0.1524) (layer "B.Cu") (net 6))
 (segment (start 175.972395 110.6424) (end 175.895 110.565005) (width 0.1524) (layer "F.Cu") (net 1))
 (segment (start 175.895 100.952) (end 176.911 99.936) (width 0.1524) (layer "F.Cu") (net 1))
 (segment (start 175.972395 117.793795) (end 176.911 118.7324) (width 0.1524) (layer "F.Cu") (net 1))
 (segment (start 175.972395 110.6424) (end 175.972395 117.793795) (width 0.1524) (layer "F.Cu") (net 1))
 (segment (start 164.9048 110.1932) (end 164.9048 108.4696) (width 0.1524) (layer "F.Cu") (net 1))
 (segment (start 175.895 110.565005) (end 175.895 100.952) (width 0.1524) (layer "F.Cu") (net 1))
 (segment (start 164.9476 110.236) (end 164.9048 110.1932) (width 0.1524) (layer "F.Cu") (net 1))
 (via (at 164.9476 110.236) (size 0.508) (drill 0.254) (layers "F.Cu" "B.Cu") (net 1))
 (via (at 175.972395 110.6424) (size 0.508) (drill 0.254) (layers "F.Cu" "B.Cu") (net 1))
 (segment (start 165.3286 110.6424) (end 164.9476 110.2614) (width 0.1524) (layer "B.Cu") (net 1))
 (segment (start 164.9476 110.2614) (end 164.9476 110.236) (width 0.1524) (layer "B.Cu") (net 1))
 (segment (start 164.9476 110.236) (end 164.9222 110.236) (width 0.1524) (layer "B.Cu") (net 1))
 (segment (start 164.9222 110.236) (end 164.9222 110.236) (width 0.1524) (layer "B.Cu") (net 1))
 (segment (start 175.972395 110.6424) (end 165.3286 110.6424) (width 0.1524) (layer "B.Cu") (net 1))
 (segment (start 170.8658 105.843) (end 171.4246 106.4018) (width 0.1524) (layer "F.Cu") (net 7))
 (segment (start 171.4246 106.4018) (end 171.4246 109.6518) (width 0.1524) (layer "F.Cu") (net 7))
 (segment (start 169.291 99.936) (end 170.8658 101.5108) (width 0.1524) (layer "F.Cu") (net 7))
 (segment (start 171.4246 109.6518) (end 171.3992 109.6772) (width 0.1524) (layer "F.Cu") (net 7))
 (segment (start 170.892395 117.131005) (end 169.291 118.7324) (width 0.1524) (layer "F.Cu") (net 7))
 (segment (start 171.4246 112.990595) (end 170.892395 113.5228) (width 0.1524) (layer "F.Cu") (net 7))
 (segment (start 171.3992 109.6772) (end 171.4246 109.7026) (width 0.1524) (layer "F.Cu") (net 7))
 (segment (start 171.4246 109.7026) (end 171.4246 112.990595) (width 0.1524) (layer "F.Cu") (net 7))
 (segment (start 170.892395 113.5228) (end 170.892395 117.131005) (width 0.1524) (layer "F.Cu") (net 7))
 (segment (start 165.9382 109.7026) (end 165.9382 108.503) (width 0.1524) (layer "F.Cu") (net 7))
 (segment (start 170.8658 101.5108) (end 170.8658 105.843) (width 0.1524) (layer "F.Cu") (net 7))
 (segment (start 165.9382 108.503) (end 165.9048 108.4696) (width 0.1524) (layer "F.Cu") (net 7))
 (via (at 165.9382 109.7026) (size 0.508) (drill 0.254) (layers "F.Cu" "B.Cu") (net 7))
 (via (at 171.3992 109.6772) (size 0.508) (drill 0.254) (layers "F.Cu" "B.Cu") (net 7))
 (segment (start 165.9382 109.7026) (end 165.9128 109.6772) (width 0.1524) (layer "B.Cu") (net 7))
 (segment (start 166.5986 109.7026) (end 165.9382 109.7026) (width 0.1524) (layer "B.Cu") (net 7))
 (segment (start 166.0398 109.601) (end 165.9382 109.7026) (width 0.1524) (layer "B.Cu") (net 7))
 (segment (start 171.3992 109.6772) (end 167.259 109.6772) (width 0.1524) (layer "B.Cu") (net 7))
 (segment (start 167.1574 109.5756) (end 166.7256 109.5756) (width 0.1524) (layer "B.Cu") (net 7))
 (segment (start 167.259 109.6772) (end 167.1574 109.5756) (width 0.1524) (layer "B.Cu") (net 7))
 (segment (start 166.7256 109.5756) (end 166.5986 109.7026) (width 0.1524) (layer "B.Cu") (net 7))
 (segment (start 159.131 99.936) (end 158.115 100.952) (width 0.1524) (layer "F.Cu") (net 15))
 (segment (start 158.115 117.7164) (end 159.131 118.7324) (width 0.1524) (layer "F.Cu") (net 15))
 (segment (start 158.115 100.952) (end 158.115 117.7164) (width 0.1524) (layer "F.Cu") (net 15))
 (segment (start 160.8328 114.0332) (end 161.671 114.8714) (width 0.1524) (layer "F.Cu") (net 14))
 (segment (start 160.8328 104.9642) (end 160.8328 114.0332) (width 0.1524) (layer "F.Cu") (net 14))
 (segment (start 161.671 104.126) (end 160.8328 104.9642) (width 0.1524) (layer "F.Cu") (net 14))
 (segment (start 154.051 104.126) (end 154.051 114.8714) (width 0.1524) (layer "F.Cu") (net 20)))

